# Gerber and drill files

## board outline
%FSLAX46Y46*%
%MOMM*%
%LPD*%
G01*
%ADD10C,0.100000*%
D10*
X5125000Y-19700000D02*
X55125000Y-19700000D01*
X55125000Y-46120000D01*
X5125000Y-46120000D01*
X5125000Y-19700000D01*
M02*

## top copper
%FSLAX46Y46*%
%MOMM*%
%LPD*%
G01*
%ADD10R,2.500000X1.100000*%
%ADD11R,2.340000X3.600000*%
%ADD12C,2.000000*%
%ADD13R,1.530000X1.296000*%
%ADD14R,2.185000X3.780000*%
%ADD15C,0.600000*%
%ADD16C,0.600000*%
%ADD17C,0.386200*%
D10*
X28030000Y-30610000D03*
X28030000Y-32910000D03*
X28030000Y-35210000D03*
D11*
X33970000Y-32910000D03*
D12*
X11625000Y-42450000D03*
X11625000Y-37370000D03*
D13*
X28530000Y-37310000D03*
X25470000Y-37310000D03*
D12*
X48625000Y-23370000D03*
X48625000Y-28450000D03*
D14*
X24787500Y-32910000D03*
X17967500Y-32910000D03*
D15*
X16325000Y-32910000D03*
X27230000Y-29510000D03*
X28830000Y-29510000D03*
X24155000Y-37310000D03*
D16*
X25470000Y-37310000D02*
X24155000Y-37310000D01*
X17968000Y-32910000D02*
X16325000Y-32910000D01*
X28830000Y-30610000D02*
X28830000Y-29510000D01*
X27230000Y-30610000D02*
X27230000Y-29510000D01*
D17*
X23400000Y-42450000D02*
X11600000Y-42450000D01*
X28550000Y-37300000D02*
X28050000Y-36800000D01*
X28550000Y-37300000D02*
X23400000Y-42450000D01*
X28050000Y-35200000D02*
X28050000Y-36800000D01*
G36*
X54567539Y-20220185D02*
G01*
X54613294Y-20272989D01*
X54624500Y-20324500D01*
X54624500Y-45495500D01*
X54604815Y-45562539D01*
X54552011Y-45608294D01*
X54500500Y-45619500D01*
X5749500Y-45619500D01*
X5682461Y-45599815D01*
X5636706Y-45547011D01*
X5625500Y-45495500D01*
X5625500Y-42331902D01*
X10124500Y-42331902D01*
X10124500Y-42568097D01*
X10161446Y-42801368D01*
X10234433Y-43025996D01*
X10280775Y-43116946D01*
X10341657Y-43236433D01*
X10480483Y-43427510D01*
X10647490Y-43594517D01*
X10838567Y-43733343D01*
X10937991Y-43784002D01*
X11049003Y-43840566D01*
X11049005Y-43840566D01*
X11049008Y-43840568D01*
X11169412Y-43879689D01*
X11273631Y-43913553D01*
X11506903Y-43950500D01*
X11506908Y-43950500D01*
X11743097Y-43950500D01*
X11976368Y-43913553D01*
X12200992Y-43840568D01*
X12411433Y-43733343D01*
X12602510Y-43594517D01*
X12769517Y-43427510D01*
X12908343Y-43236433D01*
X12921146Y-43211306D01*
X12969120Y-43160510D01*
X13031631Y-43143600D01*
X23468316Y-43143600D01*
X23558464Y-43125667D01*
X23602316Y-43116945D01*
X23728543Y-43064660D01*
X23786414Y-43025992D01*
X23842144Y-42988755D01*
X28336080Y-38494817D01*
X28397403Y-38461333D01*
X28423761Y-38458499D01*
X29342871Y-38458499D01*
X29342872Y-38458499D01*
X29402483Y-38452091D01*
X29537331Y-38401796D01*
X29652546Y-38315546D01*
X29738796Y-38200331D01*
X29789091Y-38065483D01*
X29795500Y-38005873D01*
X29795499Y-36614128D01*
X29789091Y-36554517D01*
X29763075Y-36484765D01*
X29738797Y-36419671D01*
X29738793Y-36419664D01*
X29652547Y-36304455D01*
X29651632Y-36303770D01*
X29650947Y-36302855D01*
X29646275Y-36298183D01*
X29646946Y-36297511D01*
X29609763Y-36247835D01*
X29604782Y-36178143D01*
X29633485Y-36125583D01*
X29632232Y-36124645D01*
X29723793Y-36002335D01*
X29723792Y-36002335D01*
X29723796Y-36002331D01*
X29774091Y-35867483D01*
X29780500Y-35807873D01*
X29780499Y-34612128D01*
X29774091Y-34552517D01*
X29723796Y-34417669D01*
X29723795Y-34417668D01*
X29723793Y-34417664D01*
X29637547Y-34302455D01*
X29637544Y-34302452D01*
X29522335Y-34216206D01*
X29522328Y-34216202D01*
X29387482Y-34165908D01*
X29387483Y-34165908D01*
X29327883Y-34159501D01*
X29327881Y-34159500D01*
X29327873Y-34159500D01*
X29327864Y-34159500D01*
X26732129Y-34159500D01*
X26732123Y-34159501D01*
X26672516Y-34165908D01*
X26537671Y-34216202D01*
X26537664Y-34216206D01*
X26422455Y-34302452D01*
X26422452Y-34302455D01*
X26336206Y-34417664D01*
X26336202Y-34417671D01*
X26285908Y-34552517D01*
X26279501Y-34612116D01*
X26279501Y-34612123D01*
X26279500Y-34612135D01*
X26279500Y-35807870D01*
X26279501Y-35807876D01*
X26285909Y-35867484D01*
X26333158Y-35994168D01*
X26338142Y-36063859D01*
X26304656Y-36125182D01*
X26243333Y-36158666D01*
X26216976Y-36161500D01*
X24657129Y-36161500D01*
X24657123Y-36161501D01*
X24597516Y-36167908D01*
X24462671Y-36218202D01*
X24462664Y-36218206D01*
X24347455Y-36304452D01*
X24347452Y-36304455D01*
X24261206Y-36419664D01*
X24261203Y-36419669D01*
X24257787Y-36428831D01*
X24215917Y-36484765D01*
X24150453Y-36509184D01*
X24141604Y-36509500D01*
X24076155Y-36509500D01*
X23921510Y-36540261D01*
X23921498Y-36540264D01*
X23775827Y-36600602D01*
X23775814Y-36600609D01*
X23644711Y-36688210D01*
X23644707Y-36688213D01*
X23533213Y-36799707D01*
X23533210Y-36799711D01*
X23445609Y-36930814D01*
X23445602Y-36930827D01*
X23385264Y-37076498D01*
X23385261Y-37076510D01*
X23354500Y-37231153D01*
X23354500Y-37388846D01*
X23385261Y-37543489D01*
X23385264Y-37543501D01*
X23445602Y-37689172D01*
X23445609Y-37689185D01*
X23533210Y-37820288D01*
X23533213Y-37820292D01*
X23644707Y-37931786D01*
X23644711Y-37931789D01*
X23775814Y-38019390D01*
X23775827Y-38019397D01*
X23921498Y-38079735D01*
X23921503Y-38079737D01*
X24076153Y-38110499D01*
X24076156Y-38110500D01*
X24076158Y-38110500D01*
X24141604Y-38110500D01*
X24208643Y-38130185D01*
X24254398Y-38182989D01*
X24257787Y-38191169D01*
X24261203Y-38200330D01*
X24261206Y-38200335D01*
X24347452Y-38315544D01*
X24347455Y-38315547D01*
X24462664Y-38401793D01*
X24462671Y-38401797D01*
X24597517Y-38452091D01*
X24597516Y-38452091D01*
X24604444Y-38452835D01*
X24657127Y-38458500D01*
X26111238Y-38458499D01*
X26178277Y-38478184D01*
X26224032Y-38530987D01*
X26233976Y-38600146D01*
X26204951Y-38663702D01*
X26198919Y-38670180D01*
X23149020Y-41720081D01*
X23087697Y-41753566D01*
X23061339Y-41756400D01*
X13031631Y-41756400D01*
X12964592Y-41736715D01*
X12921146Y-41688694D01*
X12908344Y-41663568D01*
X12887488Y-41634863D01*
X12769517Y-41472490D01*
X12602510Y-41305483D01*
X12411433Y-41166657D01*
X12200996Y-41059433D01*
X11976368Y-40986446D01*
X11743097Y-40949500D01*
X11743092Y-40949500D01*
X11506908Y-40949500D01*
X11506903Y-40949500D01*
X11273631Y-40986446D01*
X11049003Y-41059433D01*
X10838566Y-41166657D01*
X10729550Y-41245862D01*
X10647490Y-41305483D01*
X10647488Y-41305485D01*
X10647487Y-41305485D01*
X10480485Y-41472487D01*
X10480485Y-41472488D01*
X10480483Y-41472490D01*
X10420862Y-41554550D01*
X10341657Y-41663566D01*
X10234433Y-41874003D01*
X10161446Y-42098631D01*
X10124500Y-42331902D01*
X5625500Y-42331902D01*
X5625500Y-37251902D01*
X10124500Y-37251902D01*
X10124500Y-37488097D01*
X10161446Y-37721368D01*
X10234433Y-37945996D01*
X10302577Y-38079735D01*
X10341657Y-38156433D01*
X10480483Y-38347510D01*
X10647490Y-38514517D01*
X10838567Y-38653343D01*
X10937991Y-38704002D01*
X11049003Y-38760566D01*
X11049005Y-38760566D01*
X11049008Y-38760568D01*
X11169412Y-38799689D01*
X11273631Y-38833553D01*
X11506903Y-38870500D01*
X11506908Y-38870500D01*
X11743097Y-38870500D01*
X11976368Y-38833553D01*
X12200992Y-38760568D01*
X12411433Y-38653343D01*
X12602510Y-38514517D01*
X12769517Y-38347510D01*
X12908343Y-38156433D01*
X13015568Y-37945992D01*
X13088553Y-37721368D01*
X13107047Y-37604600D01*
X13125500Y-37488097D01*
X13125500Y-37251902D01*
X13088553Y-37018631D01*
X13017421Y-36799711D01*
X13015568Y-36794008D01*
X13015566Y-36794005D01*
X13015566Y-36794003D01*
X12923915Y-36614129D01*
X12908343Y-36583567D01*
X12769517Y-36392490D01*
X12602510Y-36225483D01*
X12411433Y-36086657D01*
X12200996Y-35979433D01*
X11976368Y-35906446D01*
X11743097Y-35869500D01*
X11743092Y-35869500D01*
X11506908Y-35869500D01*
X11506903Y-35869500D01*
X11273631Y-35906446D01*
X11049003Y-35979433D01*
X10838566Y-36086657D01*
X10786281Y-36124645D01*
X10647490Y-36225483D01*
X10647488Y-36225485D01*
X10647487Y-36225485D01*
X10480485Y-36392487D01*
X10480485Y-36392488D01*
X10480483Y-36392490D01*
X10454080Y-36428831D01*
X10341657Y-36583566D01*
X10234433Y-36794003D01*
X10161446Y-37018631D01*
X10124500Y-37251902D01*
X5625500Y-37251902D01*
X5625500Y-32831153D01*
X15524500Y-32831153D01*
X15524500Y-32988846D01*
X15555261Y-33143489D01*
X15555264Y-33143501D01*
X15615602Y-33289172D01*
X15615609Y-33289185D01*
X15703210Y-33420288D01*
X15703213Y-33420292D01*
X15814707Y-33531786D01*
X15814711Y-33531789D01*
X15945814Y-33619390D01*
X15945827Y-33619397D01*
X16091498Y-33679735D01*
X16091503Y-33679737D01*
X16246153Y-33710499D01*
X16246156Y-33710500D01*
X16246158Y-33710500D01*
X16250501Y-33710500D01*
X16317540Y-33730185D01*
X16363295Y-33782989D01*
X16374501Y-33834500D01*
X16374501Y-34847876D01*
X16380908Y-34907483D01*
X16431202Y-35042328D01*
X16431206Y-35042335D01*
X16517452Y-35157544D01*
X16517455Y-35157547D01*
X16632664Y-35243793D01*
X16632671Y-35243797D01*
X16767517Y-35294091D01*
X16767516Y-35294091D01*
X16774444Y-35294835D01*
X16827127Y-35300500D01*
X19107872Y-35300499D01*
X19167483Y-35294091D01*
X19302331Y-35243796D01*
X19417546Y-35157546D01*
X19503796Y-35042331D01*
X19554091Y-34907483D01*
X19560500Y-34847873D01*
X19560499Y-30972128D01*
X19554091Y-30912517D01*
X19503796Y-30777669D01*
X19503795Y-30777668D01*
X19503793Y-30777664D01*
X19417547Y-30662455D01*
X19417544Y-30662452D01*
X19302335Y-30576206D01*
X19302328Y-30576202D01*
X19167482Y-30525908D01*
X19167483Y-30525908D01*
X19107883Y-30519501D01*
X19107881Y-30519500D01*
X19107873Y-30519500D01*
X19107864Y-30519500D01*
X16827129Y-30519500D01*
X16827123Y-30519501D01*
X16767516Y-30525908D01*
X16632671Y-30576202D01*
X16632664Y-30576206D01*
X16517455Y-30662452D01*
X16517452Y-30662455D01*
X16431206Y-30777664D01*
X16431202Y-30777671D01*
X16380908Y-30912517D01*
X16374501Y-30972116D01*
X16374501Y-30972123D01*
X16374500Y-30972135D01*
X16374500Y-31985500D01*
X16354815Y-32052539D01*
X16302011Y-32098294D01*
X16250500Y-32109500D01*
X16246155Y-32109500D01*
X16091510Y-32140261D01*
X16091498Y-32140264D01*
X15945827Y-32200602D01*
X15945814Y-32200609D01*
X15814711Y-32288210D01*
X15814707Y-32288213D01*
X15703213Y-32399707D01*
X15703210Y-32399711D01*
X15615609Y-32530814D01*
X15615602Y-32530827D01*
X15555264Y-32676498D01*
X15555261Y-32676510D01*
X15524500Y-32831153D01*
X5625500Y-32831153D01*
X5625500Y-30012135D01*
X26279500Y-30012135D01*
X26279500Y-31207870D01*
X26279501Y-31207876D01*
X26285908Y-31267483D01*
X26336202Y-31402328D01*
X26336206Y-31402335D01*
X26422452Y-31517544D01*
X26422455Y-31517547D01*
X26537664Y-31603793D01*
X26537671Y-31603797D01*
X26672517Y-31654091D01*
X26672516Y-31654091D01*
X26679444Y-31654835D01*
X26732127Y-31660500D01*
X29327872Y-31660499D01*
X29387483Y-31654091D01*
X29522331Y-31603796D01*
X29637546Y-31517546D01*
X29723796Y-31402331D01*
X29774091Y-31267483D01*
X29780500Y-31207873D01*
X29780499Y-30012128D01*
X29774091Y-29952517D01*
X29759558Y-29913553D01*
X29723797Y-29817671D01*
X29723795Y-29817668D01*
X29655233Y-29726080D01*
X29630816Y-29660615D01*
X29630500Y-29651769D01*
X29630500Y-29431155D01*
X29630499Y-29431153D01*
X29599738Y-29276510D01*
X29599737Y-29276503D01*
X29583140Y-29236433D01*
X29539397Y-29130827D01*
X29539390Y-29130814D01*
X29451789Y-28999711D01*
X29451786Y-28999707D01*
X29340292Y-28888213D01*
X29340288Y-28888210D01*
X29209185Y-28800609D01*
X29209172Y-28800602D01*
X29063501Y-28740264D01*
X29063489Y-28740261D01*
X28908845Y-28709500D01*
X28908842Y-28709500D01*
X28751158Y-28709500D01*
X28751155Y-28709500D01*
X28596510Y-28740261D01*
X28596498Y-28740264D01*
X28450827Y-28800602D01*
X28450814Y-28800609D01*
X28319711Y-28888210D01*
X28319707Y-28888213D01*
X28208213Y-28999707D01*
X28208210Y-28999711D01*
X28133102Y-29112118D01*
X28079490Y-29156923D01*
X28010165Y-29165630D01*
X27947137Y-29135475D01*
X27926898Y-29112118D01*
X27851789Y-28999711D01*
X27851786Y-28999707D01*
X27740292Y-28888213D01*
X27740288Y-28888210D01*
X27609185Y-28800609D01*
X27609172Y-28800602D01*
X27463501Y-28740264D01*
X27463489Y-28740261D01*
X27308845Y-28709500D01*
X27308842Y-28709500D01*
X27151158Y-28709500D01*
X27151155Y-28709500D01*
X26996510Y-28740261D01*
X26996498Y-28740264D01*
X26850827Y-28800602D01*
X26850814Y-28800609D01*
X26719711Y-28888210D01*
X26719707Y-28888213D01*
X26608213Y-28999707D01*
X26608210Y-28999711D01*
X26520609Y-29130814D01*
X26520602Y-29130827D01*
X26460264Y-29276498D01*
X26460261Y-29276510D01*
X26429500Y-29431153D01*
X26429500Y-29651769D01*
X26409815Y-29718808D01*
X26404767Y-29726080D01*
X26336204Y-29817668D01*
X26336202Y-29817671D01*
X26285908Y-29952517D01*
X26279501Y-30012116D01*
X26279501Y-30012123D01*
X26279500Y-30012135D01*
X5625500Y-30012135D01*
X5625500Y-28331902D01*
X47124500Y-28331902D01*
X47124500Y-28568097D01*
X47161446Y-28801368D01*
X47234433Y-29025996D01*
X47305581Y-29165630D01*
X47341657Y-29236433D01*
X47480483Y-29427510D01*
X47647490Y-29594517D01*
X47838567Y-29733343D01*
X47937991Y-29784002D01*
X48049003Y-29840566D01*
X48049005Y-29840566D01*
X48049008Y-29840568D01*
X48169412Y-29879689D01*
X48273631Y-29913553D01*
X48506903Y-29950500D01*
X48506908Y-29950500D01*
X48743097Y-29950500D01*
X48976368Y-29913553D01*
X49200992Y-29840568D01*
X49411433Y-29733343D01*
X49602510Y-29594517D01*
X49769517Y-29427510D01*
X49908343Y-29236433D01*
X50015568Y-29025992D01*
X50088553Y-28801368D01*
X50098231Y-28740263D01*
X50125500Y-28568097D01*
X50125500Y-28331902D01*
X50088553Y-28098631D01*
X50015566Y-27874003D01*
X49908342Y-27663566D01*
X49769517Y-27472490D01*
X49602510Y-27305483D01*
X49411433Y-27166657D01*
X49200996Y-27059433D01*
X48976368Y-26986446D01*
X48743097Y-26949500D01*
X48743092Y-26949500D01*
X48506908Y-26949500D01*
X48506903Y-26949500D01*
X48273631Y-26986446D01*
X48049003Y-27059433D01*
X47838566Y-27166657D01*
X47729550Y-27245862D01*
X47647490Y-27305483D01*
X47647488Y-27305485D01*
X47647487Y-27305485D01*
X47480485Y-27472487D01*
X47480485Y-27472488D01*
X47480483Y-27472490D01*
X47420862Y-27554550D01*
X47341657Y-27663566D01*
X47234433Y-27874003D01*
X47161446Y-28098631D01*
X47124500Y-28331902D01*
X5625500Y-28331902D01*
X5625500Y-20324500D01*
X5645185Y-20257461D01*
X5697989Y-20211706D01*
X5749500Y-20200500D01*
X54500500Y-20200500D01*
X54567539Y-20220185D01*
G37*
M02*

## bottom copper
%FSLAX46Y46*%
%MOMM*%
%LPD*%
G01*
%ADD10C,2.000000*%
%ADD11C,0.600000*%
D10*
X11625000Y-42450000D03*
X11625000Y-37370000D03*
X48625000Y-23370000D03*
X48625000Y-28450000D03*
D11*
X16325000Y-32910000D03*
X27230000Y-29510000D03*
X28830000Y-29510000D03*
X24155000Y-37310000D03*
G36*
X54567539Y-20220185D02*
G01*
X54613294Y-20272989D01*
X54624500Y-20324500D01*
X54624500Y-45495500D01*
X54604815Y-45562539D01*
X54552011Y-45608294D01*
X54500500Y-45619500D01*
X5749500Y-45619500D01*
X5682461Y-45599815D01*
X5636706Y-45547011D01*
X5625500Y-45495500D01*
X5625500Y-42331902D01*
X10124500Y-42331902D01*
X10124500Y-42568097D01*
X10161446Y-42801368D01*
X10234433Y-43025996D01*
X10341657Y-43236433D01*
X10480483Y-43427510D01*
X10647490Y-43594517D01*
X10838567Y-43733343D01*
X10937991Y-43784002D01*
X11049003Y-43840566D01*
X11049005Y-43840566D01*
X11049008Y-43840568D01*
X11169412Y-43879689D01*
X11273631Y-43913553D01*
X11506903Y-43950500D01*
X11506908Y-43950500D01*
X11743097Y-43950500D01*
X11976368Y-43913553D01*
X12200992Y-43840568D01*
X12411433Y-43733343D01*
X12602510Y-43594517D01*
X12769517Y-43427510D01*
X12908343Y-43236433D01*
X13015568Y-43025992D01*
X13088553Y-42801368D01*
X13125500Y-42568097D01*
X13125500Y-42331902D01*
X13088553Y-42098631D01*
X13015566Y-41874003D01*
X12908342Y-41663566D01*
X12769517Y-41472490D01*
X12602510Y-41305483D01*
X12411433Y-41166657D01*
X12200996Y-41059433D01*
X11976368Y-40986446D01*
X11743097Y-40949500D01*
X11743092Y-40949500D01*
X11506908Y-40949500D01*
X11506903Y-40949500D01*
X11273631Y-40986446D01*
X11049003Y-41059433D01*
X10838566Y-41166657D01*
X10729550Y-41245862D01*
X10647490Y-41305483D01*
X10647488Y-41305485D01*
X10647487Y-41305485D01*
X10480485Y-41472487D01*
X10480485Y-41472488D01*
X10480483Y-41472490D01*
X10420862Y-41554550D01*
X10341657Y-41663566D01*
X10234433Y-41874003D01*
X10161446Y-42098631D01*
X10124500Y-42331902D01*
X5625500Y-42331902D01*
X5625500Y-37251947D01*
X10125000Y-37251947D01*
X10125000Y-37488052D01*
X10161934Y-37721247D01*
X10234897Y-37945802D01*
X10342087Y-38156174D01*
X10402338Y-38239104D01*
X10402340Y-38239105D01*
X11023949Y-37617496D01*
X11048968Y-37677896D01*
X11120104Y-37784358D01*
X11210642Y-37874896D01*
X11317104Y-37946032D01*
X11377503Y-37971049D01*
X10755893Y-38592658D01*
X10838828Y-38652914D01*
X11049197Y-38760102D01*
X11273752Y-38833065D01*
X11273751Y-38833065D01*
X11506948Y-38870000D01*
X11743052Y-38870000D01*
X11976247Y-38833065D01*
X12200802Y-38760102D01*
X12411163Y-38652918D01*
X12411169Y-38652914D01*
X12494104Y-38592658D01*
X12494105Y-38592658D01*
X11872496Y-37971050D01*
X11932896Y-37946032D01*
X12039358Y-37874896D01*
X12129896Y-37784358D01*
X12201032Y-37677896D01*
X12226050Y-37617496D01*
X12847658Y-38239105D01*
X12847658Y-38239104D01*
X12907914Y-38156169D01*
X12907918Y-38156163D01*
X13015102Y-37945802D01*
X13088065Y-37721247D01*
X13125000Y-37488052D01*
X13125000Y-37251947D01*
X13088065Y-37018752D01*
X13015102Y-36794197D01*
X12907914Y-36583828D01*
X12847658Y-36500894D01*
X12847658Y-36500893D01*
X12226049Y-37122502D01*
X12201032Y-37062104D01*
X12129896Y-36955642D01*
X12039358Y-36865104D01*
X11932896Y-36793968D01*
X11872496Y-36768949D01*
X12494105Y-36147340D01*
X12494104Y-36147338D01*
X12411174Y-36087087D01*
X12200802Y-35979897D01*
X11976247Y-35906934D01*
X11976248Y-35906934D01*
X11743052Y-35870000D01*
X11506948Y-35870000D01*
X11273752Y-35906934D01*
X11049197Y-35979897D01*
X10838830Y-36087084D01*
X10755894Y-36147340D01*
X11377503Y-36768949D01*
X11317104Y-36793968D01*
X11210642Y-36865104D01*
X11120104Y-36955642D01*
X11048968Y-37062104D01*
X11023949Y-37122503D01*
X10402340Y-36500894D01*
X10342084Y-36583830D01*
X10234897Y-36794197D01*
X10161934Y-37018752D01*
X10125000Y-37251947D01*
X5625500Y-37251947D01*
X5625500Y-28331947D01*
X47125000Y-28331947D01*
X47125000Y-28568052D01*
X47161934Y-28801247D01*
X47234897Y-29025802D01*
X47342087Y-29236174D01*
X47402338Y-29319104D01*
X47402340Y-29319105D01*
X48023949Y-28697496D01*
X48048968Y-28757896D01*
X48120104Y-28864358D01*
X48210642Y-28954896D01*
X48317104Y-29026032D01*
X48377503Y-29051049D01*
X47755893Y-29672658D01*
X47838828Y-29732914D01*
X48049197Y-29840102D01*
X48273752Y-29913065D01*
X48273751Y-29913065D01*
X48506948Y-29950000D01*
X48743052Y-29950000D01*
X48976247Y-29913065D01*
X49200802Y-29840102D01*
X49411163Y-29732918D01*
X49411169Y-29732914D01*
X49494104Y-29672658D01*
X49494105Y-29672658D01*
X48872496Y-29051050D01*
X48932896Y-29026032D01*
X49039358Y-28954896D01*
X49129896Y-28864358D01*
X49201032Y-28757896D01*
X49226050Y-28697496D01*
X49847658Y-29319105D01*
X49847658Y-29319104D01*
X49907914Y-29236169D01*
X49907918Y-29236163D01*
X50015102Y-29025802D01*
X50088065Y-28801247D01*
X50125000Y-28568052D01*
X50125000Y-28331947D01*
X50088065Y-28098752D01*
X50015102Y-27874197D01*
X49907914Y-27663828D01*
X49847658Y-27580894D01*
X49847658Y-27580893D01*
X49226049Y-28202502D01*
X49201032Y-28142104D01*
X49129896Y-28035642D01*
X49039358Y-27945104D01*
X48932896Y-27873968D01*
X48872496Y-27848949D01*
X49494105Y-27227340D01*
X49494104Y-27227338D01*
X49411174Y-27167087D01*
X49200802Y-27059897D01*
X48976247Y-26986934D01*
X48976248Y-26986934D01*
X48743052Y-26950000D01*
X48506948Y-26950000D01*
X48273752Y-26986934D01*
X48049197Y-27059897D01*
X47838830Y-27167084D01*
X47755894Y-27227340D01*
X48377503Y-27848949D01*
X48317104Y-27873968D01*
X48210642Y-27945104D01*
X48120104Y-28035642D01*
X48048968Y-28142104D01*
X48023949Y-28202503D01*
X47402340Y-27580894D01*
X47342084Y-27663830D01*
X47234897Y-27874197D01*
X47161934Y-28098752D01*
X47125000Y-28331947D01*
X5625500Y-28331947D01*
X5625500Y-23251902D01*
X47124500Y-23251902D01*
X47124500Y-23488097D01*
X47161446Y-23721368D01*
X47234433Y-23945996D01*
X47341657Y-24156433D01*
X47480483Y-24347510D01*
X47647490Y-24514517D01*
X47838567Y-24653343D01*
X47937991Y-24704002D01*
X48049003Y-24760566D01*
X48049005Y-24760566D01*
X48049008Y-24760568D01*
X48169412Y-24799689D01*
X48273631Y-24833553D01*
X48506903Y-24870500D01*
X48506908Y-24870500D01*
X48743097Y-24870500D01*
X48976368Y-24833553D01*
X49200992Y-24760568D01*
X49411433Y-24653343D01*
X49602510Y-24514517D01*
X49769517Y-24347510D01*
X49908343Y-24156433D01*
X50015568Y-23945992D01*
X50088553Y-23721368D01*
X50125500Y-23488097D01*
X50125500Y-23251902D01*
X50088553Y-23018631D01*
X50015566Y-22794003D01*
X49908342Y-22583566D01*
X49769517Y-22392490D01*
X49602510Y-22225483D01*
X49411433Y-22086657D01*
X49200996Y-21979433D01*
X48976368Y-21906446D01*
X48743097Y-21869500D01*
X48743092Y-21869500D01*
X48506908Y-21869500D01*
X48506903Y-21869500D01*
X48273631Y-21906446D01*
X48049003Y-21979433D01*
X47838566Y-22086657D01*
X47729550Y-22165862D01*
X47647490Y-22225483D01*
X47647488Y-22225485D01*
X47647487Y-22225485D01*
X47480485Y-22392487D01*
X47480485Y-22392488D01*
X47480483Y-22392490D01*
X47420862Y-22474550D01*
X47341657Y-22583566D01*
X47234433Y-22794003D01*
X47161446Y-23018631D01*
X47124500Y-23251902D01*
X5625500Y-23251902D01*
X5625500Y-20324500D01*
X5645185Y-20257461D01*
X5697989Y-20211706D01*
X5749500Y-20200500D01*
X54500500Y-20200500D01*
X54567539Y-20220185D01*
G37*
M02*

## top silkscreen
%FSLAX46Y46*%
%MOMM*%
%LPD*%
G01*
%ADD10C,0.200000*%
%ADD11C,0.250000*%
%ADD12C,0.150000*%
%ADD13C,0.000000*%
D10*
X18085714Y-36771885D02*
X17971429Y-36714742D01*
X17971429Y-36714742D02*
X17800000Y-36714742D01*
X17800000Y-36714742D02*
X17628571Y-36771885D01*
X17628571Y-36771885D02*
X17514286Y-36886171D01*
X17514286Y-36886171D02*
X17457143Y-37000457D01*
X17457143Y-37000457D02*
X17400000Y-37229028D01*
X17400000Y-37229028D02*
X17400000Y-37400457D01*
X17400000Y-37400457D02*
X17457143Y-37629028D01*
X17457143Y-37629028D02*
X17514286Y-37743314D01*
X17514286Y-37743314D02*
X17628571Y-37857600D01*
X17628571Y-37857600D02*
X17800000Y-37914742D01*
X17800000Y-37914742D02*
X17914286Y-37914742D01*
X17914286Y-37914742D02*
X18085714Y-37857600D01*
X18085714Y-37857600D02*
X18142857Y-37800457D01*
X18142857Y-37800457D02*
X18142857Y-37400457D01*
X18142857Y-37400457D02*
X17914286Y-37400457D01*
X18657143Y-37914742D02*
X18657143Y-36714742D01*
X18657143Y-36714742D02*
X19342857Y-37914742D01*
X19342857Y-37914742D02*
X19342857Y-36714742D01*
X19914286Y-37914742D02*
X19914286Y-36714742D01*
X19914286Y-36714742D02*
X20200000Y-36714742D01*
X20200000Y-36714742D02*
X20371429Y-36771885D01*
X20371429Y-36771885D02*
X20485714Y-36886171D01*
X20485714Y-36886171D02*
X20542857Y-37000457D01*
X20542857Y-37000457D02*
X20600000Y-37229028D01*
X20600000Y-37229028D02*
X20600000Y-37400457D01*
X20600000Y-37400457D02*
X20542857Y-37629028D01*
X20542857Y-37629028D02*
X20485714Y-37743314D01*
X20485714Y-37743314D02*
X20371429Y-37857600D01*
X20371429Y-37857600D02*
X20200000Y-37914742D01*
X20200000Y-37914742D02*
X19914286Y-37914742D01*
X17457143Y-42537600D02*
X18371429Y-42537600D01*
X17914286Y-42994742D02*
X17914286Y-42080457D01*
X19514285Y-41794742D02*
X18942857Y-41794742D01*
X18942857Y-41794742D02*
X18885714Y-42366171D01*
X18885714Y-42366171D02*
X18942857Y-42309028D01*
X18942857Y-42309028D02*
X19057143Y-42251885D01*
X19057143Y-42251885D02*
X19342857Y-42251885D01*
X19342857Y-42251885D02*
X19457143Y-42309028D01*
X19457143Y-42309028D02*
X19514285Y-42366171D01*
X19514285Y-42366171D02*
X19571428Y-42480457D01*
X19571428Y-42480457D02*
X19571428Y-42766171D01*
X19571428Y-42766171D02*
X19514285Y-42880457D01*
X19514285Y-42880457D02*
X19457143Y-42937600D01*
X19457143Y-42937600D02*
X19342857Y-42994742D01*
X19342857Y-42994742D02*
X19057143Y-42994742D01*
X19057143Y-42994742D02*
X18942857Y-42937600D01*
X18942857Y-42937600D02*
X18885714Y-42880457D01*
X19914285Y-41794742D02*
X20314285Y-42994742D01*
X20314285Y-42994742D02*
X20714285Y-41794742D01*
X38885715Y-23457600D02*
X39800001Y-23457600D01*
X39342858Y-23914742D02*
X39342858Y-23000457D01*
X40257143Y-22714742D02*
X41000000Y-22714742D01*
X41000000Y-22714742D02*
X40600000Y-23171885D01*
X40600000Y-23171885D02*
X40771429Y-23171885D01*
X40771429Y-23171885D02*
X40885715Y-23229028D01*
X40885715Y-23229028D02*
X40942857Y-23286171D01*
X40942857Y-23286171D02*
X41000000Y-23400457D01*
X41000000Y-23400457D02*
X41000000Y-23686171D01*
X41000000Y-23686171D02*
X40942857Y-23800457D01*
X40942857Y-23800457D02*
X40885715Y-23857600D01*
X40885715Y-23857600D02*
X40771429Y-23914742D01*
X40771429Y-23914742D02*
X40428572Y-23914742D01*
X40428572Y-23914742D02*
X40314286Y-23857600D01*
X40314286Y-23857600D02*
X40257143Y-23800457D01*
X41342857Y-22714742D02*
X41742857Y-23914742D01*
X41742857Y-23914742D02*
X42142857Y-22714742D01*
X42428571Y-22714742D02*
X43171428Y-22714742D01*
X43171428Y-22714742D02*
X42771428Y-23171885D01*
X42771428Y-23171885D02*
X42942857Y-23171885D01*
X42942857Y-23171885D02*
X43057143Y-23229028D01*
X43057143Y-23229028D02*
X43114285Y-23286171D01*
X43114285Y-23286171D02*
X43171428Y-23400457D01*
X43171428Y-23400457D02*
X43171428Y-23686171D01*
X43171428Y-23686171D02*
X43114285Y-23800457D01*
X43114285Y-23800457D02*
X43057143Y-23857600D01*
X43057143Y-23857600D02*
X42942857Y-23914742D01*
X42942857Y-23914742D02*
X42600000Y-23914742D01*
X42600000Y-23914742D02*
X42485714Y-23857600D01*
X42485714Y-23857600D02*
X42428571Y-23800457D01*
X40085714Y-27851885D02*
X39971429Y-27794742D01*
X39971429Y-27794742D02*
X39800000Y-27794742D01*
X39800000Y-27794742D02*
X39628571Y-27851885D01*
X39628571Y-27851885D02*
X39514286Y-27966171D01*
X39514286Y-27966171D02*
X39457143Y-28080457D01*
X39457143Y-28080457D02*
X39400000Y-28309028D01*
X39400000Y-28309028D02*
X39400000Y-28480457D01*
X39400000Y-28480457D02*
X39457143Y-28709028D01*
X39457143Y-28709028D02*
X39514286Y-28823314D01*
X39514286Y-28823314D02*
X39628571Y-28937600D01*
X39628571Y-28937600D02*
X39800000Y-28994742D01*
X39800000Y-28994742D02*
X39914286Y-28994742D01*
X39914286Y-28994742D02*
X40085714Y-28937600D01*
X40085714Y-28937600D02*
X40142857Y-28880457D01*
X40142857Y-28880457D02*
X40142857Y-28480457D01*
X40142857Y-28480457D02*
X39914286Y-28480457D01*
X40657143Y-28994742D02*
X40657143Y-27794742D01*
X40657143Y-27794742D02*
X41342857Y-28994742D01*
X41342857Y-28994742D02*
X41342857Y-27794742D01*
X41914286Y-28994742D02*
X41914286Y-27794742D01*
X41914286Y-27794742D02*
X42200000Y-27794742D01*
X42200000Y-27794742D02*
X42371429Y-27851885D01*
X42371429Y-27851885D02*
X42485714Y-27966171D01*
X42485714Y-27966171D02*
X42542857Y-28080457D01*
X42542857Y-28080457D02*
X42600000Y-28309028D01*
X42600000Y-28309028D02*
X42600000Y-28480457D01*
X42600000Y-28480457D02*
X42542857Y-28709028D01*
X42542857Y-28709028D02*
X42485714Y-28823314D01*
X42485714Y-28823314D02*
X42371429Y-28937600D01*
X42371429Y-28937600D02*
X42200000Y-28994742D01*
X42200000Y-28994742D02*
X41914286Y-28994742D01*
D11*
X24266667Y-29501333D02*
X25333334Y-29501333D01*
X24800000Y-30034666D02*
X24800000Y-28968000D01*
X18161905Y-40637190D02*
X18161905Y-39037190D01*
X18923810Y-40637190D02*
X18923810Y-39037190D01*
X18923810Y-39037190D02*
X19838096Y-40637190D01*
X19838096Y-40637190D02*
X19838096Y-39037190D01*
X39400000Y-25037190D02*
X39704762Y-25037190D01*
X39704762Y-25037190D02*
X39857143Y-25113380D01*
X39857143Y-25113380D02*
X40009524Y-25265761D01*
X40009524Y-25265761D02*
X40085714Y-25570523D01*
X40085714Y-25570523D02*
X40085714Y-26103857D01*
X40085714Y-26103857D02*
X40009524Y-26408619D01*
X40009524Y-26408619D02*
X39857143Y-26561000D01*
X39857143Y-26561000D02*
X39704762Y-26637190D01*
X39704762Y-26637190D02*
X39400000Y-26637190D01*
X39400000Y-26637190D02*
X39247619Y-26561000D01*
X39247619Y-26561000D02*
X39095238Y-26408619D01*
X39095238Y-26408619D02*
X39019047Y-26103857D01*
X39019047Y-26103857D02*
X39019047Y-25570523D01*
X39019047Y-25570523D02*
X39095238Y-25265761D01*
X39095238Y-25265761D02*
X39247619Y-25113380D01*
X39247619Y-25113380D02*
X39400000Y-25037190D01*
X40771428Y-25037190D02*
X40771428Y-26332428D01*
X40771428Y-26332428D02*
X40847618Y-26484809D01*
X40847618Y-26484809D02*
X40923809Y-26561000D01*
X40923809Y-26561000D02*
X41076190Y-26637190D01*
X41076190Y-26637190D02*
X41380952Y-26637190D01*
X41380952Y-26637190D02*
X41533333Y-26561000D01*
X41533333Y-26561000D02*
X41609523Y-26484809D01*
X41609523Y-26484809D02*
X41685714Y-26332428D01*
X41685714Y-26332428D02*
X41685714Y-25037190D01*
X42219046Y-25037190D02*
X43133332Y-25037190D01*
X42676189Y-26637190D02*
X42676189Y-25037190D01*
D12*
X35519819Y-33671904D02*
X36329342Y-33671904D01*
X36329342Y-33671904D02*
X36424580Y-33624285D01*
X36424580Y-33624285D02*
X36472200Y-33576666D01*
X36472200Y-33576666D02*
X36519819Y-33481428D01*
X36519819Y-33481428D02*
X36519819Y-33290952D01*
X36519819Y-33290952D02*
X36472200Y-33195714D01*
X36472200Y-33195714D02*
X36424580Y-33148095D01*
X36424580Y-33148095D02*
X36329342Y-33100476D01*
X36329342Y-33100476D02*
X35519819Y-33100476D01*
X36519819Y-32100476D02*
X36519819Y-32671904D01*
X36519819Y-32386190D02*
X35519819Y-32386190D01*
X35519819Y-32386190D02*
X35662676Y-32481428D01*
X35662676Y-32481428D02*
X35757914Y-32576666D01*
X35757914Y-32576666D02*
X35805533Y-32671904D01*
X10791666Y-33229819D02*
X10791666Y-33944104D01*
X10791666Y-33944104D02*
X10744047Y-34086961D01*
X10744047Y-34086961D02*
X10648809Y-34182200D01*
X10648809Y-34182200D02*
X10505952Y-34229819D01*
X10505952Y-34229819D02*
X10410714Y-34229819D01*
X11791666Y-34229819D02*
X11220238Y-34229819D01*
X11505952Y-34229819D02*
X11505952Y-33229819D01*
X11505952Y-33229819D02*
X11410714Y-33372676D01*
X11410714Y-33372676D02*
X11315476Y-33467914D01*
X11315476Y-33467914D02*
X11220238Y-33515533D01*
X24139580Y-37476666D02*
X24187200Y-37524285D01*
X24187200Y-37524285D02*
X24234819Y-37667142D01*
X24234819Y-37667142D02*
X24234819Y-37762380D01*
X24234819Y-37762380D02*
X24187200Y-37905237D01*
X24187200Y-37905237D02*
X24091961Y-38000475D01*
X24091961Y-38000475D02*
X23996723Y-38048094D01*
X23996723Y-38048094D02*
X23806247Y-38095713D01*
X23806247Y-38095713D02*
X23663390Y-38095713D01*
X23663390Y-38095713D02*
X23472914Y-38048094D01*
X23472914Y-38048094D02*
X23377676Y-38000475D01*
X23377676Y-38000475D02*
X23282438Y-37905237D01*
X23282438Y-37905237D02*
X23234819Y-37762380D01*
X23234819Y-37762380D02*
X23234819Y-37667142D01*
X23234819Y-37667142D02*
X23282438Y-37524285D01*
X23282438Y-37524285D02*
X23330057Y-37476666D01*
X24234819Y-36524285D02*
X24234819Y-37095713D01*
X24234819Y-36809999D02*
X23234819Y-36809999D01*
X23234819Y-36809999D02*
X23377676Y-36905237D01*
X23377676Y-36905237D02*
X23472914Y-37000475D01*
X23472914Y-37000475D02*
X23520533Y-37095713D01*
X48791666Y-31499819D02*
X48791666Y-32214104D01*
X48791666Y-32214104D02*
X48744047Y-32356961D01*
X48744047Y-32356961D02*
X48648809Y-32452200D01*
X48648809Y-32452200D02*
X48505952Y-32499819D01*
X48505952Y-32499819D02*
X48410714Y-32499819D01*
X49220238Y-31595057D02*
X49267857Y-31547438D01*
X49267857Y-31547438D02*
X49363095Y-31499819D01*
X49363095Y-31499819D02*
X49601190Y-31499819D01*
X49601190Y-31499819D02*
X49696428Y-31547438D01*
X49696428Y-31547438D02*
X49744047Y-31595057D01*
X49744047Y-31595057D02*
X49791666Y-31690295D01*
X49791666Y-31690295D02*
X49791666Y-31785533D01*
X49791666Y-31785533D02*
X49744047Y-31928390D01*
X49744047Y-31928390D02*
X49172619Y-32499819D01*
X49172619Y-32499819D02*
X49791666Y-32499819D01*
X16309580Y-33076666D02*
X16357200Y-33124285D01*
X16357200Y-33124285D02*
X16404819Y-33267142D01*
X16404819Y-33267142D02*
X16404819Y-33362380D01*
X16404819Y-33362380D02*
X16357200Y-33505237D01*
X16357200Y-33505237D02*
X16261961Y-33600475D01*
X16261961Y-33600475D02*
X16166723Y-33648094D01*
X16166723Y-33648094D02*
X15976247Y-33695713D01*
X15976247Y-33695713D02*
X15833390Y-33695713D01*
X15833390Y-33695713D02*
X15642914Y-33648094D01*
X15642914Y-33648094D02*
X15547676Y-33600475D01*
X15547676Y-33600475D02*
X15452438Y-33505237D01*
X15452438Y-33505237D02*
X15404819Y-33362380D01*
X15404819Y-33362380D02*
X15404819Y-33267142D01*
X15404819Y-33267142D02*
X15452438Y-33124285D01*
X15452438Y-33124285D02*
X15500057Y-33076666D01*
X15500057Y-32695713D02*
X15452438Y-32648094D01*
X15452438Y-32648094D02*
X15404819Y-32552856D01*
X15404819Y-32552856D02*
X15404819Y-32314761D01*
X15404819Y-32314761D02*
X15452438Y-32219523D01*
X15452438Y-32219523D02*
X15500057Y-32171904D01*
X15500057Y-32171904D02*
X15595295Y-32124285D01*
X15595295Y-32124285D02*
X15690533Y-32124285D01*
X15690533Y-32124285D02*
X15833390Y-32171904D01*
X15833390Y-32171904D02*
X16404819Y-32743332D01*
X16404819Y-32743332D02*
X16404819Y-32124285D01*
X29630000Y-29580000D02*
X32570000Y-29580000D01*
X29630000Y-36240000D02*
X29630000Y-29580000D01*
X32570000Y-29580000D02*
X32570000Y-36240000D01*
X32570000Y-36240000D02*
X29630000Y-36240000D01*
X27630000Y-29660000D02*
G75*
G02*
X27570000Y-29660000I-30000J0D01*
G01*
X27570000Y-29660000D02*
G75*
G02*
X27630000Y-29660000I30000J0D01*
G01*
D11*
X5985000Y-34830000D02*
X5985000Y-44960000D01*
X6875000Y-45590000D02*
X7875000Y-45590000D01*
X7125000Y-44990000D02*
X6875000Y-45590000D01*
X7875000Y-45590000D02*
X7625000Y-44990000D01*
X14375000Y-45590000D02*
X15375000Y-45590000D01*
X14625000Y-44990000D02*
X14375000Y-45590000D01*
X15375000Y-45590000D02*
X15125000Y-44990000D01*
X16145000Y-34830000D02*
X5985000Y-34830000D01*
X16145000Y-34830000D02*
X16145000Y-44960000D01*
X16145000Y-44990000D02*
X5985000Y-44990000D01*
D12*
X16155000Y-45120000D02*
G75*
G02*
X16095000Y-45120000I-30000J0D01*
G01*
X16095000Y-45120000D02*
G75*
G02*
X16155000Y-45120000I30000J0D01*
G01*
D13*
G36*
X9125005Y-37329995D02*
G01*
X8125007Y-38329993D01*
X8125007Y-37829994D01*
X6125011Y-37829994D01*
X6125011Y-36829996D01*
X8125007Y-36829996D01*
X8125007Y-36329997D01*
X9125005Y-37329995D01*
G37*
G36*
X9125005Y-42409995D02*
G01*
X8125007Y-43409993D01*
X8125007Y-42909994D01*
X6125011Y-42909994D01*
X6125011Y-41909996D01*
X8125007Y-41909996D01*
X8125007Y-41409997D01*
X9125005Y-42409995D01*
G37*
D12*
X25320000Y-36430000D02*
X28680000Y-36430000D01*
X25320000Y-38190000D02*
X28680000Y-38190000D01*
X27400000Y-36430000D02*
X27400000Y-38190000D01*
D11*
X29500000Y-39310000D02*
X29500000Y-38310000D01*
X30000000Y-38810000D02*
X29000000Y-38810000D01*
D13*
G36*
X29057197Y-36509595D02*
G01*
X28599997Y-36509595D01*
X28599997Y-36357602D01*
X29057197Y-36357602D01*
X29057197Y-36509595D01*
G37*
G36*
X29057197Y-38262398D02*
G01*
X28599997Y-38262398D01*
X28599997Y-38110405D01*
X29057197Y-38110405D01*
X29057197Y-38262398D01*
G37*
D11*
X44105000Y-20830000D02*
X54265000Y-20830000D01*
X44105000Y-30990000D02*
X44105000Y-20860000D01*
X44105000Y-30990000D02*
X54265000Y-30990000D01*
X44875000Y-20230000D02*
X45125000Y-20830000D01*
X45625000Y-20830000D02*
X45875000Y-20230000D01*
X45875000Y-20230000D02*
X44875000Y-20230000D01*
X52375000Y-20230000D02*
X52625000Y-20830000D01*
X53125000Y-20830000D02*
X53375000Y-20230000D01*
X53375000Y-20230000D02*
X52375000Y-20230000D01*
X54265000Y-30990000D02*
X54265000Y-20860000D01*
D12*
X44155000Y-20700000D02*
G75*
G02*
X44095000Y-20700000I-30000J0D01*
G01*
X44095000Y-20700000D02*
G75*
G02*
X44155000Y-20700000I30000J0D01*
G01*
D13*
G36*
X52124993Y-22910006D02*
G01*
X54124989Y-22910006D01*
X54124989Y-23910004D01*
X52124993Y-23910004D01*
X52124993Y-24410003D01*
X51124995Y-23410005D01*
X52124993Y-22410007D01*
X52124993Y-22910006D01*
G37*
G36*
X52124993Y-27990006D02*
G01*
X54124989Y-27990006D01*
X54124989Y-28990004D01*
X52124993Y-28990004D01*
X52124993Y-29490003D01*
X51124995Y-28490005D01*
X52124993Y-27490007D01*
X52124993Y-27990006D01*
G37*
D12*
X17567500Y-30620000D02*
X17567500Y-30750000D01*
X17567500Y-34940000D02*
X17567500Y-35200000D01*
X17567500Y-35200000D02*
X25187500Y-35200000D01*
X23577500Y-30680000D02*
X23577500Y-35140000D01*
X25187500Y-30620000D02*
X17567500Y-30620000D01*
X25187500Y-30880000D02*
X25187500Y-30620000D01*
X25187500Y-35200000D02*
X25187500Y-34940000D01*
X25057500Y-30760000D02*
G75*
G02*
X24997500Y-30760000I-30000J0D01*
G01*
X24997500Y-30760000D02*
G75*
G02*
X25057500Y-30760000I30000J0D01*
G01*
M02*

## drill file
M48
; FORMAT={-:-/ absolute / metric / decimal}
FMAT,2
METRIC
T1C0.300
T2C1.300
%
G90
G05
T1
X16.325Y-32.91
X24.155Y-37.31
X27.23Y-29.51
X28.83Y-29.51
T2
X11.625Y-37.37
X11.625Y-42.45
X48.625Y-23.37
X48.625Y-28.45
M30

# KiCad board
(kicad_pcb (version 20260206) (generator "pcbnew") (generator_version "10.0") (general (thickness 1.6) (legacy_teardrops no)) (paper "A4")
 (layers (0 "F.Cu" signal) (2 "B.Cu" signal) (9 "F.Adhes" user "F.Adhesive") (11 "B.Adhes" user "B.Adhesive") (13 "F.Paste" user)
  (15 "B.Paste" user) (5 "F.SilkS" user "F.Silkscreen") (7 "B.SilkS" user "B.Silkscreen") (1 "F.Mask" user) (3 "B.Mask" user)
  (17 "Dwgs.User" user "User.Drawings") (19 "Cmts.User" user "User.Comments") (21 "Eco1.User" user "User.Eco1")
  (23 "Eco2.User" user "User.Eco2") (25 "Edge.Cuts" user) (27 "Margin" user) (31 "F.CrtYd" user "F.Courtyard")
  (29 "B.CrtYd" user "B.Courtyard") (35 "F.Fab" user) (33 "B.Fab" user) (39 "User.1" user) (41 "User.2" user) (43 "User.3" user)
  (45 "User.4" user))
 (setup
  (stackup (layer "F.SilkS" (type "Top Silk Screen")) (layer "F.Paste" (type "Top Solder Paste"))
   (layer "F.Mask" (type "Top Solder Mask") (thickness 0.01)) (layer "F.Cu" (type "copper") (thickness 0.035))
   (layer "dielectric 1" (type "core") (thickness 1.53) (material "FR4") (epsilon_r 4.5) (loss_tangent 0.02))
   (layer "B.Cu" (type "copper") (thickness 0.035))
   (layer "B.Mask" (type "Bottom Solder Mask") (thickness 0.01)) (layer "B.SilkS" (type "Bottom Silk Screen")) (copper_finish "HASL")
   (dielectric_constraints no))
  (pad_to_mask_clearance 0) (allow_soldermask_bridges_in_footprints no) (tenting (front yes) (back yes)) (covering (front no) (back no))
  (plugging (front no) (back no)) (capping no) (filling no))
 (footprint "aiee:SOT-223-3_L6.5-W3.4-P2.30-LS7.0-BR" (layer "F.Cu") (at 31 32.91 180)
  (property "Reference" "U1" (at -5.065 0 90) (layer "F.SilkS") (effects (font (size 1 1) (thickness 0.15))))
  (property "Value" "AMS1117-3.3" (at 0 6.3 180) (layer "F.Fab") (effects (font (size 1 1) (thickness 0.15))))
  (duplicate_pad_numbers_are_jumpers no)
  (fp_line (start 1.37 3.33) (end -1.57 3.33) (stroke (width 0.15) (type solid)) (layer "F.SilkS"))
  (fp_line (start 1.37 -3.33) (end 1.37 3.33) (stroke (width 0.15) (type solid)) (layer "F.SilkS"))
  (fp_line (start -1.57 3.33) (end -1.57 -3.33) (stroke (width 0.15) (type solid)) (layer "F.SilkS"))
  (fp_line (start -1.57 -3.33) (end 1.37 -3.33) (stroke (width 0.15) (type solid)) (layer "F.SilkS"))
  (fp_circle (center 3.4 3.25) (end 3.43 3.25) (stroke (width 0.15) (type solid)) (fill no) (layer "F.SilkS"))
  (pad "1" smd rect (at 2.97 2.3 180) (size 2.5 1.1) (layers "F.Cu" "F.Mask" "F.Paste") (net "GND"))
  (pad "2" smd rect (at 2.97 0 180) (size 2.5 1.1) (layers "F.Cu" "F.Mask" "F.Paste") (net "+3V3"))
  (pad "3" smd rect (at 2.97 -2.3 180) (size 2.5 1.1) (layers "F.Cu" "F.Mask" "F.Paste") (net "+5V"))
  (pad "4" smd rect (at -2.97 0 180) (size 2.34 3.6) (layers "F.Cu" "F.Mask" "F.Paste") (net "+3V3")))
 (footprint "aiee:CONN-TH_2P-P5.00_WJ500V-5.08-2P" (layer "F.Cu") (at 11.625 39.91 90)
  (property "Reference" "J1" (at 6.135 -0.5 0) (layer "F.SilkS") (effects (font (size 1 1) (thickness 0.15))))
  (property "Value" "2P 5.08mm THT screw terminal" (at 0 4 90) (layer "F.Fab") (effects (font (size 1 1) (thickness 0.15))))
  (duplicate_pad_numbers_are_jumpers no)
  (fp_line (start 5.08 -5.64) (end -5.05 -5.64) (stroke (width 0.25) (type solid)) (layer "F.SilkS"))
  (fp_line (start -5.68 -4.75) (end -5.68 -3.75) (stroke (width 0.25) (type solid)) (layer "F.SilkS"))
  (fp_line (start -5.08 -4.5) (end -5.68 -4.75) (stroke (width 0.25) (type solid)) (layer "F.SilkS"))
  (fp_line (start -5.68 -3.75) (end -5.08 -4) (stroke (width 0.25) (type solid)) (layer "F.SilkS"))
  (fp_line (start -5.68 2.75) (end -5.68 3.75) (stroke (width 0.25) (type solid)) (layer "F.SilkS"))
  (fp_line (start -5.08 3) (end -5.68 2.75) (stroke (width 0.25) (type solid)) (layer "F.SilkS"))
  (fp_line (start -5.68 3.75) (end -5.08 3.5) (stroke (width 0.25) (type solid)) (layer "F.SilkS"))
  (fp_line (start 5.08 4.52) (end 5.08 -5.64) (stroke (width 0.25) (type solid)) (layer "F.SilkS"))
  (fp_line (start 5.08 4.52) (end -5.05 4.52) (stroke (width 0.25) (type solid)) (layer "F.SilkS"))
  (fp_line (start -5.08 4.52) (end -5.08 -5.64) (stroke (width 0.25) (type solid)) (layer "F.SilkS"))
  (fp_circle (center -5.21 4.5) (end -5.18 4.5) (stroke (width 0.15) (type solid)) (fill no) (layer "F.SilkS"))
  (fp_poly
   (pts (xy 2.080006 -5.499989) (xy 3.080004 -5.499989) (xy 3.080004 -3.499993) (xy 3.580003 -3.499993) (xy 2.580005 -2.499995)
    (xy 1.580007 -3.499993) (xy 2.080006 -3.499993) (xy 2.080006 -5.499989))
   (stroke (width 0) (type solid)) (fill yes) (layer "F.SilkS"))
  (fp_poly
   (pts (xy -2.999994 -5.499989) (xy -1.999996 -5.499989) (xy -1.999996 -3.499993) (xy -1.499997 -3.499993) (xy -2.499995 -2.499995)
    (xy -3.499993 -3.499993) (xy -2.999994 -3.499993) (xy -2.999994 -5.499989))
   (stroke (width 0) (type solid)) (fill yes) (layer "F.SilkS"))
  (pad "1" thru_hole circle (at -2.54 0 270) (size 2 2) (drill 1.300022) (layers "*.Cu" "*.Mask") (remove_unused_layers no) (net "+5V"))
  (pad "2" thru_hole circle (at 2.54 0 270) (size 2 2) (drill 1.300022) (layers "*.Cu" "*.Mask") (remove_unused_layers no) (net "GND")))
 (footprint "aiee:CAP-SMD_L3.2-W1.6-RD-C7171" (layer "F.Cu") (at 27 37.31 180)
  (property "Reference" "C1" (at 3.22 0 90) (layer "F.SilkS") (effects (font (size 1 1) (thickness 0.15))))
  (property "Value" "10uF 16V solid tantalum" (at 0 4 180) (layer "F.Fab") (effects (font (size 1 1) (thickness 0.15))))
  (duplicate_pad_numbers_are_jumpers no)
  (fp_line (start 1.68 0.88) (end -1.68 0.88) (stroke (width 0.15) (type solid)) (layer "F.SilkS"))
  (fp_line (start 1.68 -0.88) (end -1.68 -0.88) (stroke (width 0.15) (type solid)) (layer "F.SilkS"))
  (fp_line (start -0.4 0.88) (end -0.4 -0.88) (stroke (width 0.15) (type solid)) (layer "F.SilkS"))
  (fp_line (start -2.5 -2) (end -2.5 -1) (stroke (width 0.25) (type solid)) (layer "F.SilkS"))
  (fp_line (start -3 -1.5) (end -2 -1.5) (stroke (width 0.25) (type solid)) (layer "F.SilkS"))
  (fp_poly
   (pts (xy -1.599997 0.952398) (xy -1.599997 0.800405) (xy -2.057197 0.800405) (xy -2.057197 0.952398) (xy -1.599997 0.952398))
   (stroke (width 0) (type solid)) (fill yes) (layer "F.SilkS"))
  (fp_poly
   (pts (xy -1.599997 -0.952398) (xy -1.599997 -0.800405) (xy -2.057197 -0.800405) (xy -2.057197 -0.952398) (xy -1.599997 -0.952398))
   (stroke (width 0) (type solid)) (fill yes) (layer "F.SilkS"))
  (pad "1" smd rect (at -1.53 0) (size 1.53 1.296) (layers "F.Cu" "F.Mask" "F.Paste") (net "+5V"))
  (pad "2" smd rect (at 1.53 0) (size 1.53 1.296) (layers "F.Cu" "F.Mask" "F.Paste") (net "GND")))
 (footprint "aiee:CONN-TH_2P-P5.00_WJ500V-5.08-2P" (layer "F.Cu") (at 48.625 25.91 -90)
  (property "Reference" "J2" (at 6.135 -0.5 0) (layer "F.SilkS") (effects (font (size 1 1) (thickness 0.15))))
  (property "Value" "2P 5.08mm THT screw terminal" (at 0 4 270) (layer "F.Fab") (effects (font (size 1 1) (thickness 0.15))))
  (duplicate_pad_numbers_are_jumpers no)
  (fp_line (start -5.08 4.52) (end -5.08 -5.64) (stroke (width 0.25) (type solid)) (layer "F.SilkS"))
  (fp_line (start 5.08 4.52) (end -5.05 4.52) (stroke (width 0.25) (type solid)) (layer "F.SilkS"))
  (fp_line (start 5.08 4.52) (end 5.08 -5.64) (stroke (width 0.25) (type solid)) (layer "F.SilkS"))
  (fp_line (start -5.68 3.75) (end -5.08 3.5) (stroke (width 0.25) (type solid)) (layer "F.SilkS"))
  (fp_line (start -5.08 3) (end -5.68 2.75) (stroke (width 0.25) (type solid)) (layer "F.SilkS"))
  (fp_line (start -5.68 2.75) (end -5.68 3.75) (stroke (width 0.25) (type solid)) (layer "F.SilkS"))
  (fp_line (start -5.68 -3.75) (end -5.08 -4) (stroke (width 0.25) (type solid)) (layer "F.SilkS"))
  (fp_line (start -5.08 -4.5) (end -5.68 -4.75) (stroke (width 0.25) (type solid)) (layer "F.SilkS"))
  (fp_line (start -5.68 -4.75) (end -5.68 -3.75) (stroke (width 0.25) (type solid)) (layer "F.SilkS"))
  (fp_line (start 5.08 -5.64) (end -5.05 -5.64) (stroke (width 0.25) (type solid)) (layer "F.SilkS"))
  (fp_circle (center -5.21 4.5) (end -5.18 4.5) (stroke (width 0.15) (type solid)) (fill no) (layer "F.SilkS"))
  (fp_poly
   (pts (xy -2.999994 -5.499989) (xy -1.999996 -5.499989) (xy -1.999996 -3.499993) (xy -1.499997 -3.499993) (xy -2.499995 -2.499995)
    (xy -3.499993 -3.499993) (xy -2.999994 -3.499993) (xy -2.999994 -5.499989))
   (stroke (width 0) (type solid)) (fill yes) (layer "F.SilkS"))
  (fp_poly
   (pts (xy 2.080006 -5.499989) (xy 3.080004 -5.499989) (xy 3.080004 -3.499993) (xy 3.580003 -3.499993) (xy 2.580005 -2.499995)
    (xy 1.580007 -3.499993) (xy 2.080006 -3.499993) (xy 2.080006 -5.499989))
   (stroke (width 0) (type solid)) (fill yes) (layer "F.SilkS"))
  (pad "1" thru_hole circle (at -2.54 0 90) (size 2 2) (drill 1.300022) (layers "*.Cu" "*.Mask") (remove_unused_layers no) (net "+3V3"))
  (pad "2" thru_hole circle (at 2.54 0 90) (size 2 2) (drill 1.300022) (layers "*.Cu" "*.Mask") (remove_unused_layers no) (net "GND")))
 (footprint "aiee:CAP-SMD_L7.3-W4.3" (layer "F.Cu") (at 21.3775 32.91)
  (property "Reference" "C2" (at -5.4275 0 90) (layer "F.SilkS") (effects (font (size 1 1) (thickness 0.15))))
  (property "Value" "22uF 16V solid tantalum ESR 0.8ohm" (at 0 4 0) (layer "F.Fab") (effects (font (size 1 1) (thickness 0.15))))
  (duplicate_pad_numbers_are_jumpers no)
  (fp_line (start -3.81 -2.29) (end -3.81 -2.16) (stroke (width 0.15) (type solid)) (layer "F.SilkS"))
  (fp_line (start -3.81 2.03) (end -3.81 2.29) (stroke (width 0.15) (type solid)) (layer "F.SilkS"))
  (fp_line (start -3.81 2.29) (end 3.81 2.29) (stroke (width 0.15) (type solid)) (layer "F.SilkS"))
  (fp_line (start 2.2 -2.23) (end 2.2 2.23) (stroke (width 0.15) (type solid)) (layer "F.SilkS"))
  (fp_line (start 3.81 -2.29) (end -3.81 -2.29) (stroke (width 0.15) (type solid)) (layer "F.SilkS"))
  (fp_line (start 3.81 -2.03) (end 3.81 -2.29) (stroke (width 0.15) (type solid)) (layer "F.SilkS"))
  (fp_line (start 3.81 2.29) (end 3.81 2.03) (stroke (width 0.15) (type solid)) (layer "F.SilkS"))
  (fp_circle (center 3.65 -2.15) (end 3.68 -2.15) (stroke (width 0.15) (type solid)) (fill no) (layer "F.SilkS"))
  (pad "1" smd rect (at 3.41 0 180) (size 2.185 3.78) (layers "F.Cu" "F.Mask" "F.Paste") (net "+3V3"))
  (pad "2" smd rect (at -3.41 0 180) (size 2.185 3.78) (layers "F.Cu" "F.Mask" "F.Paste") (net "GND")))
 (gr_rect (start 5.125 19.7) (end 55.125 46.12) (stroke (width 0.1) (type default)) (fill no) (layer "Edge.Cuts"))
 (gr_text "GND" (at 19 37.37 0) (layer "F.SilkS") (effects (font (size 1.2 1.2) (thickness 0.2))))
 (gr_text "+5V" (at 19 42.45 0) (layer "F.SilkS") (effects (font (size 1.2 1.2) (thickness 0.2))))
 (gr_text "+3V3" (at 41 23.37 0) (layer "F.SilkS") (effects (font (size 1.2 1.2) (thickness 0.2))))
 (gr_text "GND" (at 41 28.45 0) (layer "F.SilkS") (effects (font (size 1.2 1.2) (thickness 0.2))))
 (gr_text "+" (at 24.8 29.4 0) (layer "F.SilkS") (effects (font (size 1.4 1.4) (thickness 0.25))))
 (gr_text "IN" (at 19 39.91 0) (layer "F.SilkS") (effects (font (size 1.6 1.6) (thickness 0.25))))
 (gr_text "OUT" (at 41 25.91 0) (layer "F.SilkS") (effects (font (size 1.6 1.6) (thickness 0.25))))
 (segment (start 25.47 37.31) (end 24.155 37.31) (width 0.6) (layer "F.Cu") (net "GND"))
 (segment (start 17.968 32.91) (end 16.325 32.91) (width 0.6) (layer "F.Cu") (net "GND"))
 (segment (start 28.83 30.61) (end 28.83 29.51) (width 0.6) (layer "F.Cu") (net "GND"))
 (segment (start 27.23 30.61) (end 27.23 29.51) (width 0.6) (layer "F.Cu") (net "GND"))
 (via (at 16.325 32.91) (size 0.6) (drill 0.3) (layers "F.Cu" "B.Cu") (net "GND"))
 (via (at 27.23 29.51) (size 0.6) (drill 0.3) (layers "F.Cu" "B.Cu") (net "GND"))
 (via (at 28.83 29.51) (size 0.6) (drill 0.3) (layers "F.Cu" "B.Cu") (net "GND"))
 (via (at 24.155 37.31) (size 0.6) (drill 0.3) (layers "F.Cu" "B.Cu") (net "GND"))
 (segment (start 23.4 42.45) (end 11.6 42.45) (width 0.3862) (layer "F.Cu") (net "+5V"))
 (segment (start 28.55 37.3) (end 28.05 36.8) (width 0.3862) (layer "F.Cu") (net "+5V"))
 (segment (start 28.55 37.3) (end 23.4 42.45) (width 0.3862) (layer "F.Cu") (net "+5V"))
 (segment (start 28.05 35.2) (end 28.05 36.8) (width 0.3862) (layer "F.Cu") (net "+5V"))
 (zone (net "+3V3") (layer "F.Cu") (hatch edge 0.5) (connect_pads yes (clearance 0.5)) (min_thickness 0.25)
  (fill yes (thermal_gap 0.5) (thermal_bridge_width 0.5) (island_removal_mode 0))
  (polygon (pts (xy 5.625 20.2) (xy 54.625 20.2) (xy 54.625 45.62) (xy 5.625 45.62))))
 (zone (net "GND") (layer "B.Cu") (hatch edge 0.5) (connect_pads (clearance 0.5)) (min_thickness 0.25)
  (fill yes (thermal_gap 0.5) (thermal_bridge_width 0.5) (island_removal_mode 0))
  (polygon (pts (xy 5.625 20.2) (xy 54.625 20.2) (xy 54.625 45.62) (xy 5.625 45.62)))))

